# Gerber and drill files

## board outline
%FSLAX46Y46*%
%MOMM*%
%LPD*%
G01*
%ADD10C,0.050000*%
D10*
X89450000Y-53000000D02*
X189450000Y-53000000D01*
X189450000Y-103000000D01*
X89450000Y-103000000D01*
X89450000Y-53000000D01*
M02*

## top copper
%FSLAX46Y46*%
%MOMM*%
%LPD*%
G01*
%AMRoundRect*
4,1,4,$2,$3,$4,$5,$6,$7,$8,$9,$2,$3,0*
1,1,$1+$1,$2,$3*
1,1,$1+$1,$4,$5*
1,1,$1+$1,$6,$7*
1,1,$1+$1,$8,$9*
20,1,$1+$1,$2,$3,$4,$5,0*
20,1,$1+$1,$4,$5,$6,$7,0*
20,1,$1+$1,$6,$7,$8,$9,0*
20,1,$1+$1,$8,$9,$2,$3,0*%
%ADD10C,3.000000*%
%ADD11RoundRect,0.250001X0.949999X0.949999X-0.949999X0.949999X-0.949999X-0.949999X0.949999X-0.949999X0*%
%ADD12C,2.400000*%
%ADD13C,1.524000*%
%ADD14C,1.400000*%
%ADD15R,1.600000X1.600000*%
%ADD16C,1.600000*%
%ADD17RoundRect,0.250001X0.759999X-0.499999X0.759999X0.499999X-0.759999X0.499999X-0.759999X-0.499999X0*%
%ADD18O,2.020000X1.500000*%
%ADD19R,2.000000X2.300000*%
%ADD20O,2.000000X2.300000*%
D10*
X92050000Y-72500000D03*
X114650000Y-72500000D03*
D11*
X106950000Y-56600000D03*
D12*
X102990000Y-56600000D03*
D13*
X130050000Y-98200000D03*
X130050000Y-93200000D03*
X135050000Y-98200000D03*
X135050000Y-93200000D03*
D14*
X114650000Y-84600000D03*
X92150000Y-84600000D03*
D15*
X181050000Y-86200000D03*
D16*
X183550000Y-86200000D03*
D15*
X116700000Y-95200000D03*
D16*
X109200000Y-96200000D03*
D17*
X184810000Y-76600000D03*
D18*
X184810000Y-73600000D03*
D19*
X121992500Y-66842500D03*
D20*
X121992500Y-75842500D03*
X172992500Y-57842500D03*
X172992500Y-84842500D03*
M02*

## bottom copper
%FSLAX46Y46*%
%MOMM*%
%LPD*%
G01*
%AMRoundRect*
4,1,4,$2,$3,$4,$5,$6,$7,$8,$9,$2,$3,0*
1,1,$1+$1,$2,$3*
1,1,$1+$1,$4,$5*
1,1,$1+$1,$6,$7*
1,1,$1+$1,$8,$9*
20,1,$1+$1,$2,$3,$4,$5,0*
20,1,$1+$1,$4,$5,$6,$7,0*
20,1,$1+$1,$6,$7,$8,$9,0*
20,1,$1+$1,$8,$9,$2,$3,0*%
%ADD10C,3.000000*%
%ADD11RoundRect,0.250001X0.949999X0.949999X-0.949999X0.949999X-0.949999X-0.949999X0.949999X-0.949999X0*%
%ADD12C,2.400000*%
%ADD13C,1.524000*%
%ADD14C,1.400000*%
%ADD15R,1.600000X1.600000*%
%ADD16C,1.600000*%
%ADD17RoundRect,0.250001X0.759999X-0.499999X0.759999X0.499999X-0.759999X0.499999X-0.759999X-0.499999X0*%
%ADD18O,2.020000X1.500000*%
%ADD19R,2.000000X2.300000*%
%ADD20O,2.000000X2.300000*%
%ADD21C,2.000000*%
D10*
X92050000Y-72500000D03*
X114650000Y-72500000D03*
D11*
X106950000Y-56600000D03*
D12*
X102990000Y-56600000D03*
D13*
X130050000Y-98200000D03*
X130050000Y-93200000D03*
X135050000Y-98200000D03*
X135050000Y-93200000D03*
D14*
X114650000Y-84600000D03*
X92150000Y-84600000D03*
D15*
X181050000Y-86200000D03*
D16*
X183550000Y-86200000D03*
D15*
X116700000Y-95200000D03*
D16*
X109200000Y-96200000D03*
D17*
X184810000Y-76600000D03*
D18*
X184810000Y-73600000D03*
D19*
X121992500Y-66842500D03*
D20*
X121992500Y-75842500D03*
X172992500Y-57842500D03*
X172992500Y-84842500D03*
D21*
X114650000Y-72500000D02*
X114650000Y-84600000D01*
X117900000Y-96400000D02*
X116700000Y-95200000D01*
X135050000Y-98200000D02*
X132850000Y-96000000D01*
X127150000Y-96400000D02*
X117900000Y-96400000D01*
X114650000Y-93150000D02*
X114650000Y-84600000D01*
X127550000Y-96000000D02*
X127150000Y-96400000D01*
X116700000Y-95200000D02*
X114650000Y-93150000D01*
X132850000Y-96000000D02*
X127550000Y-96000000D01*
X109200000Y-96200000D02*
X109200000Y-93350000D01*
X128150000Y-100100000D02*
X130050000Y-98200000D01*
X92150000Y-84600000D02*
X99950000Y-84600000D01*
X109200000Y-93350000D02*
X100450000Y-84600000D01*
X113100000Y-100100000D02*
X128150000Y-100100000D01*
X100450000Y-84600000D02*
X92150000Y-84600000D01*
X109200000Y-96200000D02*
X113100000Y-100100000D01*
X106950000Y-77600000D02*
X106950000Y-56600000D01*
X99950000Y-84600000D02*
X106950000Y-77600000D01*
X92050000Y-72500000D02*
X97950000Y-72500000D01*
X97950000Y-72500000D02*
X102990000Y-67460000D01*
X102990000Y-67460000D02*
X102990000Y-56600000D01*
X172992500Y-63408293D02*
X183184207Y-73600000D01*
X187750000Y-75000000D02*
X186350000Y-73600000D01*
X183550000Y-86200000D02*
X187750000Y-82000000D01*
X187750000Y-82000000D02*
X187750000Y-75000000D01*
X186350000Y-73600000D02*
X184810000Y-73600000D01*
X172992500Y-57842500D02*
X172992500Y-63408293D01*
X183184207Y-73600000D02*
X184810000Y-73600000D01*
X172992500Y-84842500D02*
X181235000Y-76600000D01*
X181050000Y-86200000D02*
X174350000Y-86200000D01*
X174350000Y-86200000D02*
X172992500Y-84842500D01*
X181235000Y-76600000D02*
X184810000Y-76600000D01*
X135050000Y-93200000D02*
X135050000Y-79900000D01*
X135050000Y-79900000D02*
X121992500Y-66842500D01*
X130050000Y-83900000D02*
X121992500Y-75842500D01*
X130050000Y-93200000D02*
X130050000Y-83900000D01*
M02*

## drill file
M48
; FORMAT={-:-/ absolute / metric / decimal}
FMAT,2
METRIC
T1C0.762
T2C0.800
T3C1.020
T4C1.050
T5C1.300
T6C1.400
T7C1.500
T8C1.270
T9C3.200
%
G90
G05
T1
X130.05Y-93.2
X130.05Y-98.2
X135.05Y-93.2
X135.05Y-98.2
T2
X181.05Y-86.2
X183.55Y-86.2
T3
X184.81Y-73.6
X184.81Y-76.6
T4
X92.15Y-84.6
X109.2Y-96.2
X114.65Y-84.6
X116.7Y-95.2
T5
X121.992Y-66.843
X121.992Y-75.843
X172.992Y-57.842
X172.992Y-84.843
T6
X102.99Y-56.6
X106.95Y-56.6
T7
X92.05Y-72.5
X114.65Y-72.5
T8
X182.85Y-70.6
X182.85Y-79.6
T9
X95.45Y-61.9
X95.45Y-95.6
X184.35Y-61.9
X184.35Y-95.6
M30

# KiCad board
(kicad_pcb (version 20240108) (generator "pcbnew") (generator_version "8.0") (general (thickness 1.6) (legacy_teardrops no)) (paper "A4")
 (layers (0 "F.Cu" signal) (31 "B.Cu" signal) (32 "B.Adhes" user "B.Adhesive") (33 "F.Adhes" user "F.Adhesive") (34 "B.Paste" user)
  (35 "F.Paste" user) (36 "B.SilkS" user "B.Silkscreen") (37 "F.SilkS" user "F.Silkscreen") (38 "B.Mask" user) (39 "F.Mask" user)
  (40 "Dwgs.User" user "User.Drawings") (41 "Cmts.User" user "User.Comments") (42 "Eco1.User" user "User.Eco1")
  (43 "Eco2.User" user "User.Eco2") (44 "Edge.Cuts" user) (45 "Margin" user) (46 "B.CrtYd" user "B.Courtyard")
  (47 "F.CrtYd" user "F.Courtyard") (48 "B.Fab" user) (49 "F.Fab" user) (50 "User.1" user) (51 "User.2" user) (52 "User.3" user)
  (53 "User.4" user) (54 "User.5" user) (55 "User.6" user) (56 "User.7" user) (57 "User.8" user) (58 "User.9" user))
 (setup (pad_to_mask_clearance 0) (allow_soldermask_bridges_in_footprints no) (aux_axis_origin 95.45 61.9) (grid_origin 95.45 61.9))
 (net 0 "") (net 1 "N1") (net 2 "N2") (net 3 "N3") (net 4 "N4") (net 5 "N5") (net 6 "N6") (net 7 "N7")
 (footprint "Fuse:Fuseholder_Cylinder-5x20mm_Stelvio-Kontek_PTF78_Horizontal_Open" (layer "F.Cu") (at 92.05 72.5)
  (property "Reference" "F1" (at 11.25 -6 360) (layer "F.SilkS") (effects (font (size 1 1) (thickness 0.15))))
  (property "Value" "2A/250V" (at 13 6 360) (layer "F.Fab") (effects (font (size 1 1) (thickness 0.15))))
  (pad "1" thru_hole circle (at 0 0) (size 3 3) (drill 1.5) (layers "*.Cu" "*.Mask") (remove_unused_layers no) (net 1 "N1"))
  (pad "2" thru_hole circle (at 22.6 0) (size 3 3) (drill 1.5) (layers "*.Cu" "*.Mask") (remove_unused_layers no) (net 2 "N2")))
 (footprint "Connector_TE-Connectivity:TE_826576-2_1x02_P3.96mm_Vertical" (layer "F.Cu") (at 106.95 56.6 180)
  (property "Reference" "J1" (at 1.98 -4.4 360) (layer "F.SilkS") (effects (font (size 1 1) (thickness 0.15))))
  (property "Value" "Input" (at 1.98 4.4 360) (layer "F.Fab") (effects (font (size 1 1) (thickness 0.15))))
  (pad "1" thru_hole roundrect (at 0 0 180) (size 2.4 2.4) (drill 1.4) (layers "*.Cu" "*.Mask") (remove_unused_layers no)
   (roundrect_rratio 0.104167) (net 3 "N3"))
  (pad "2" thru_hole circle (at 3.96 0 180) (size 2.4 2.4) (drill 1.4) (layers "*.Cu" "*.Mask") (remove_unused_layers no) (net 1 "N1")))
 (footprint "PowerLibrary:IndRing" (layer "F.Cu") (at 132.55 95.7 180)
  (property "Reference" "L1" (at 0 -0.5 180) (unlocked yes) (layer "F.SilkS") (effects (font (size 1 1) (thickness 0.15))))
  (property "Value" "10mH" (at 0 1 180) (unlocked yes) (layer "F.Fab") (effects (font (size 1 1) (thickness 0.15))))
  (pad "1" thru_hole circle (at 2.5 -2.5 180) (size 1.524 1.524) (drill 0.762) (layers "*.Cu" "*.Mask") (remove_unused_layers no)
   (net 3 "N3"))
  (pad "2" thru_hole circle (at 2.5 2.5 180) (size 1.524 1.524) (drill 0.762) (layers "*.Cu" "*.Mask") (remove_unused_layers no)
   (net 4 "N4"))
  (pad "3" thru_hole circle (at -2.5 -2.5 180) (size 1.524 1.524) (drill 0.762) (layers "*.Cu" "*.Mask") (remove_unused_layers no)
   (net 2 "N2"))
  (pad "4" thru_hole circle (at -2.5 2.5 180) (size 1.524 1.524) (drill 0.762) (layers "*.Cu" "*.Mask") (remove_unused_layers no)
   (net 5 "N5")))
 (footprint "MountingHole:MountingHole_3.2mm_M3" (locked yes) (layer "F.Cu") (at 184.35 95.6)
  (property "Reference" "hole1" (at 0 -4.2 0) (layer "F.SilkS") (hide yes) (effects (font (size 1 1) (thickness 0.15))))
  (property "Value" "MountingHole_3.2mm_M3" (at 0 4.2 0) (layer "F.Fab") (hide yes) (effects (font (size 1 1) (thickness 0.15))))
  (pad "" np_thru_hole circle (at 0 0) (size 3.2 3.2) (drill 3.2) (layers "*.Cu" "*.Mask")))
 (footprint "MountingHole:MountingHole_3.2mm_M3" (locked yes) (layer "F.Cu") (at 95.45 61.9)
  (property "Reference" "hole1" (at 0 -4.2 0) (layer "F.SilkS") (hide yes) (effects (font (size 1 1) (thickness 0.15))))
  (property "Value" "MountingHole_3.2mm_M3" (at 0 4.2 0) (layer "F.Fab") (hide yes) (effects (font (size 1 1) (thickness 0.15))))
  (pad "" np_thru_hole circle (at 0 0) (size 3.2 3.2) (drill 3.2) (layers "*.Cu" "*.Mask")))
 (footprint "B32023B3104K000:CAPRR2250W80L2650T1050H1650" (layer "F.Cu") (at 103.4 84.6 180)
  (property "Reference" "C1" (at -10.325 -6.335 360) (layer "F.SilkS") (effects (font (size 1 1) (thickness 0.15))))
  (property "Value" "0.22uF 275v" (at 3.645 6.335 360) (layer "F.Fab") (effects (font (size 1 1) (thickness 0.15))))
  (pad "1" thru_hole circle (at -11.25 0 180) (size 1.4 1.4) (drill 1.05) (layers "*.Cu" "*.Mask") (remove_unused_layers no) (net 2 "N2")
   (solder_mask_margin 0.102))
  (pad "2" thru_hole circle (at 11.25 0 180) (size 1.4 1.4) (drill 1.05) (layers "*.Cu" "*.Mask") (remove_unused_layers no) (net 3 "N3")
   (solder_mask_margin 0.102)))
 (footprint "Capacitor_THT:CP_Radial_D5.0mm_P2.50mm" (layer "F.Cu") (at 181.05 86.2)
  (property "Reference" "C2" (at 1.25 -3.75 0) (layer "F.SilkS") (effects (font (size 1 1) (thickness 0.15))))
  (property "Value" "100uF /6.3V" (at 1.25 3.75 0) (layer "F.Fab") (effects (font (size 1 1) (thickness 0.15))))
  (pad "1" thru_hole rect (at 0 0) (size 1.6 1.6) (drill 0.8) (layers "*.Cu" "*.Mask") (remove_unused_layers no) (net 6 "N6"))
  (pad "2" thru_hole circle (at 2.5 0) (size 1.6 1.6) (drill 0.8) (layers "*.Cu" "*.Mask") (remove_unused_layers no) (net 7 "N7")))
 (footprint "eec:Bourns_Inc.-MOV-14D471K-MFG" (layer "F.Cu") (at 112.95 95.7 180)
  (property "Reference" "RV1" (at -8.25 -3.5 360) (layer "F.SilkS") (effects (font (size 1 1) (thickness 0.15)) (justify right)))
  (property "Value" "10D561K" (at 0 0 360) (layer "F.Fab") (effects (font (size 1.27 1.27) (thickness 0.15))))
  (pad "1" thru_hole rect (at -3.75 0.5 180) (size 1.6 1.6) (drill 1.05) (layers "*.Cu") (remove_unused_layers no) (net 2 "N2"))
  (pad "2" thru_hole circle (at 3.75 -0.5 180) (size 1.6 1.6) (drill 1.05) (layers "*.Cu") (remove_unused_layers no) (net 3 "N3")))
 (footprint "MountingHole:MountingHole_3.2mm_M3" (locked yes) (layer "F.Cu") (at 184.35 61.9)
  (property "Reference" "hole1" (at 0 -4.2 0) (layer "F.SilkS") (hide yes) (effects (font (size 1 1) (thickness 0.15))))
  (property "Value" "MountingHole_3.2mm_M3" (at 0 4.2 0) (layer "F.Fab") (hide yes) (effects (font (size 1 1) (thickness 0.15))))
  (pad "" np_thru_hole circle (at 0 0) (size 3.2 3.2) (drill 3.2) (layers "*.Cu" "*.Mask")))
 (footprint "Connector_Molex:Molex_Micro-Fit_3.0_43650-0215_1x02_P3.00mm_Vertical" (layer "F.Cu") (at 184.81 76.6 90)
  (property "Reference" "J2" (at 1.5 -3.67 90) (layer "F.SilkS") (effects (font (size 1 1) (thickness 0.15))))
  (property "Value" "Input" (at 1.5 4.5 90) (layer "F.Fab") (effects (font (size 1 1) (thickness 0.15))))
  (pad "" np_thru_hole circle (at -3 -1.96 90) (size 1.27 1.27) (drill 1.27) (layers "*.Cu" "*.Mask"))
  (pad "" np_thru_hole circle (at 6 -1.96 90) (size 1.27 1.27) (drill 1.27) (layers "*.Cu" "*.Mask"))
  (pad "1" thru_hole roundrect (at 0 0 90) (size 1.5 2.02) (drill 1.02) (layers "*.Cu" "*.Mask") (remove_unused_layers no)
   (roundrect_rratio 0.166667) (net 6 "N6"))
  (pad "2" thru_hole oval (at 3 0 90) (size 1.5 2.02) (drill 1.02) (layers "*.Cu" "*.Mask") (remove_unused_layers no) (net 7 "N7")))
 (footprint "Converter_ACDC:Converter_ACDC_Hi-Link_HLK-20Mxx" (layer "F.Cu") (at 121.9925 66.8425)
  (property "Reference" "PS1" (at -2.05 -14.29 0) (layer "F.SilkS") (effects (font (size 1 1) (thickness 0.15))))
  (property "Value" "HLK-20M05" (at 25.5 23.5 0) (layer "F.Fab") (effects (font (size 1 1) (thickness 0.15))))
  (pad "1" thru_hole rect (at 0 0) (size 2 2.3) (drill 1.3) (layers "*.Cu" "*.Mask") (remove_unused_layers no) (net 5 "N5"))
  (pad "2" thru_hole oval (at 0 9) (size 2 2.3) (drill 1.3) (layers "*.Cu" "*.Mask") (remove_unused_layers no) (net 4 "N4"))
  (pad "3" thru_hole oval (at 51 -9) (size 2 2.3) (drill 1.3) (layers "*.Cu" "*.Mask") (remove_unused_layers no) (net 7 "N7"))
  (pad "4" thru_hole oval (at 51 18) (size 2 2.3) (drill 1.3) (layers "*.Cu" "*.Mask") (remove_unused_layers no) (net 6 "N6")))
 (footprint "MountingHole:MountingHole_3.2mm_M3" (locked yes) (layer "F.Cu") (at 95.45 95.6)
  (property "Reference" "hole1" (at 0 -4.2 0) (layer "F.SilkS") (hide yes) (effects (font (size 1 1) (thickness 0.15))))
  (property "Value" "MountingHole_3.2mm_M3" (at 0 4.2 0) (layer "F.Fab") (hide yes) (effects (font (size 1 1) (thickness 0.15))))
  (pad "" np_thru_hole circle (at 0 0) (size 3.2 3.2) (drill 3.2) (layers "*.Cu" "*.Mask")))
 (gr_rect (start 89.45 53) (end 189.45 103) (stroke (width 0.05) (type default)) (fill none) (layer "Edge.Cuts"))
 (segment (start 114.65 72.5) (end 114.65 84.6) (width 2) (layer "B.Cu") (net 2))
 (segment (start 117.9 96.4) (end 116.7 95.2) (width 2) (layer "B.Cu") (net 2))
 (segment (start 135.05 98.2) (end 132.85 96) (width 2) (layer "B.Cu") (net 2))
 (segment (start 127.15 96.4) (end 117.9 96.4) (width 2) (layer "B.Cu") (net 2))
 (segment (start 114.65 93.15) (end 114.65 84.6) (width 2) (layer "B.Cu") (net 2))
 (segment (start 127.55 96) (end 127.15 96.4) (width 2) (layer "B.Cu") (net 2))
 (segment (start 116.7 95.2) (end 114.65 93.15) (width 2) (layer "B.Cu") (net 2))
 (segment (start 132.85 96) (end 127.55 96) (width 2) (layer "B.Cu") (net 2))
 (segment (start 109.2 96.2) (end 109.2 93.35) (width 2) (layer "B.Cu") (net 3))
 (segment (start 128.15 100.1) (end 130.05 98.2) (width 2) (layer "B.Cu") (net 3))
 (segment (start 92.15 84.6) (end 99.95 84.6) (width 2) (layer "B.Cu") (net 3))
 (segment (start 109.2 93.35) (end 100.45 84.6) (width 2) (layer "B.Cu") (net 3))
 (segment (start 113.1 100.1) (end 128.15 100.1) (width 2) (layer "B.Cu") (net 3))
 (segment (start 100.45 84.6) (end 92.15 84.6) (width 2) (layer "B.Cu") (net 3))
 (segment (start 109.2 96.2) (end 113.1 100.1) (width 2) (layer "B.Cu") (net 3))
 (segment (start 106.95 77.6) (end 106.95 56.6) (width 2) (layer "B.Cu") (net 3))
 (segment (start 99.95 84.6) (end 106.95 77.6) (width 2) (layer "B.Cu") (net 3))
 (segment (start 92.05 72.5) (end 97.95 72.5) (width 2) (layer "B.Cu") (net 1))
 (segment (start 97.95 72.5) (end 102.99 67.46) (width 2) (layer "B.Cu") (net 1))
 (segment (start 102.99 67.46) (end 102.99 56.6) (width 2) (layer "B.Cu") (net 1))
 (segment (start 172.9925 63.408293) (end 183.184207 73.6) (width 2) (layer "B.Cu") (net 7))
 (segment (start 187.75 75) (end 186.35 73.6) (width 2) (layer "B.Cu") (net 7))
 (segment (start 183.55 86.2) (end 187.75 82) (width 2) (layer "B.Cu") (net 7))
 (segment (start 187.75 82) (end 187.75 75) (width 2) (layer "B.Cu") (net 7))
 (segment (start 186.35 73.6) (end 184.81 73.6) (width 2) (layer "B.Cu") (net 7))
 (segment (start 172.9925 57.8425) (end 172.9925 63.408293) (width 2) (layer "B.Cu") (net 7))
 (segment (start 183.184207 73.6) (end 184.81 73.6) (width 2) (layer "B.Cu") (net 7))
 (segment (start 172.9925 84.8425) (end 181.235 76.6) (width 2) (layer "B.Cu") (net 6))
 (segment (start 181.05 86.2) (end 174.35 86.2) (width 2) (layer "B.Cu") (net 6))
 (segment (start 174.35 86.2) (end 172.9925 84.8425) (width 2) (layer "B.Cu") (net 6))
 (segment (start 181.235 76.6) (end 184.81 76.6) (width 2) (layer "B.Cu") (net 6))
 (segment (start 135.05 93.2) (end 135.05 79.9) (width 2) (layer "B.Cu") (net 5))
 (segment (start 135.05 79.9) (end 121.9925 66.8425) (width 2) (layer "B.Cu") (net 5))
 (segment (start 130.05 83.9) (end 121.9925 75.8425) (width 2) (layer "B.Cu") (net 4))
 (segment (start 130.05 93.2) (end 130.05 83.9) (width 2) (layer "B.Cu") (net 4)))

